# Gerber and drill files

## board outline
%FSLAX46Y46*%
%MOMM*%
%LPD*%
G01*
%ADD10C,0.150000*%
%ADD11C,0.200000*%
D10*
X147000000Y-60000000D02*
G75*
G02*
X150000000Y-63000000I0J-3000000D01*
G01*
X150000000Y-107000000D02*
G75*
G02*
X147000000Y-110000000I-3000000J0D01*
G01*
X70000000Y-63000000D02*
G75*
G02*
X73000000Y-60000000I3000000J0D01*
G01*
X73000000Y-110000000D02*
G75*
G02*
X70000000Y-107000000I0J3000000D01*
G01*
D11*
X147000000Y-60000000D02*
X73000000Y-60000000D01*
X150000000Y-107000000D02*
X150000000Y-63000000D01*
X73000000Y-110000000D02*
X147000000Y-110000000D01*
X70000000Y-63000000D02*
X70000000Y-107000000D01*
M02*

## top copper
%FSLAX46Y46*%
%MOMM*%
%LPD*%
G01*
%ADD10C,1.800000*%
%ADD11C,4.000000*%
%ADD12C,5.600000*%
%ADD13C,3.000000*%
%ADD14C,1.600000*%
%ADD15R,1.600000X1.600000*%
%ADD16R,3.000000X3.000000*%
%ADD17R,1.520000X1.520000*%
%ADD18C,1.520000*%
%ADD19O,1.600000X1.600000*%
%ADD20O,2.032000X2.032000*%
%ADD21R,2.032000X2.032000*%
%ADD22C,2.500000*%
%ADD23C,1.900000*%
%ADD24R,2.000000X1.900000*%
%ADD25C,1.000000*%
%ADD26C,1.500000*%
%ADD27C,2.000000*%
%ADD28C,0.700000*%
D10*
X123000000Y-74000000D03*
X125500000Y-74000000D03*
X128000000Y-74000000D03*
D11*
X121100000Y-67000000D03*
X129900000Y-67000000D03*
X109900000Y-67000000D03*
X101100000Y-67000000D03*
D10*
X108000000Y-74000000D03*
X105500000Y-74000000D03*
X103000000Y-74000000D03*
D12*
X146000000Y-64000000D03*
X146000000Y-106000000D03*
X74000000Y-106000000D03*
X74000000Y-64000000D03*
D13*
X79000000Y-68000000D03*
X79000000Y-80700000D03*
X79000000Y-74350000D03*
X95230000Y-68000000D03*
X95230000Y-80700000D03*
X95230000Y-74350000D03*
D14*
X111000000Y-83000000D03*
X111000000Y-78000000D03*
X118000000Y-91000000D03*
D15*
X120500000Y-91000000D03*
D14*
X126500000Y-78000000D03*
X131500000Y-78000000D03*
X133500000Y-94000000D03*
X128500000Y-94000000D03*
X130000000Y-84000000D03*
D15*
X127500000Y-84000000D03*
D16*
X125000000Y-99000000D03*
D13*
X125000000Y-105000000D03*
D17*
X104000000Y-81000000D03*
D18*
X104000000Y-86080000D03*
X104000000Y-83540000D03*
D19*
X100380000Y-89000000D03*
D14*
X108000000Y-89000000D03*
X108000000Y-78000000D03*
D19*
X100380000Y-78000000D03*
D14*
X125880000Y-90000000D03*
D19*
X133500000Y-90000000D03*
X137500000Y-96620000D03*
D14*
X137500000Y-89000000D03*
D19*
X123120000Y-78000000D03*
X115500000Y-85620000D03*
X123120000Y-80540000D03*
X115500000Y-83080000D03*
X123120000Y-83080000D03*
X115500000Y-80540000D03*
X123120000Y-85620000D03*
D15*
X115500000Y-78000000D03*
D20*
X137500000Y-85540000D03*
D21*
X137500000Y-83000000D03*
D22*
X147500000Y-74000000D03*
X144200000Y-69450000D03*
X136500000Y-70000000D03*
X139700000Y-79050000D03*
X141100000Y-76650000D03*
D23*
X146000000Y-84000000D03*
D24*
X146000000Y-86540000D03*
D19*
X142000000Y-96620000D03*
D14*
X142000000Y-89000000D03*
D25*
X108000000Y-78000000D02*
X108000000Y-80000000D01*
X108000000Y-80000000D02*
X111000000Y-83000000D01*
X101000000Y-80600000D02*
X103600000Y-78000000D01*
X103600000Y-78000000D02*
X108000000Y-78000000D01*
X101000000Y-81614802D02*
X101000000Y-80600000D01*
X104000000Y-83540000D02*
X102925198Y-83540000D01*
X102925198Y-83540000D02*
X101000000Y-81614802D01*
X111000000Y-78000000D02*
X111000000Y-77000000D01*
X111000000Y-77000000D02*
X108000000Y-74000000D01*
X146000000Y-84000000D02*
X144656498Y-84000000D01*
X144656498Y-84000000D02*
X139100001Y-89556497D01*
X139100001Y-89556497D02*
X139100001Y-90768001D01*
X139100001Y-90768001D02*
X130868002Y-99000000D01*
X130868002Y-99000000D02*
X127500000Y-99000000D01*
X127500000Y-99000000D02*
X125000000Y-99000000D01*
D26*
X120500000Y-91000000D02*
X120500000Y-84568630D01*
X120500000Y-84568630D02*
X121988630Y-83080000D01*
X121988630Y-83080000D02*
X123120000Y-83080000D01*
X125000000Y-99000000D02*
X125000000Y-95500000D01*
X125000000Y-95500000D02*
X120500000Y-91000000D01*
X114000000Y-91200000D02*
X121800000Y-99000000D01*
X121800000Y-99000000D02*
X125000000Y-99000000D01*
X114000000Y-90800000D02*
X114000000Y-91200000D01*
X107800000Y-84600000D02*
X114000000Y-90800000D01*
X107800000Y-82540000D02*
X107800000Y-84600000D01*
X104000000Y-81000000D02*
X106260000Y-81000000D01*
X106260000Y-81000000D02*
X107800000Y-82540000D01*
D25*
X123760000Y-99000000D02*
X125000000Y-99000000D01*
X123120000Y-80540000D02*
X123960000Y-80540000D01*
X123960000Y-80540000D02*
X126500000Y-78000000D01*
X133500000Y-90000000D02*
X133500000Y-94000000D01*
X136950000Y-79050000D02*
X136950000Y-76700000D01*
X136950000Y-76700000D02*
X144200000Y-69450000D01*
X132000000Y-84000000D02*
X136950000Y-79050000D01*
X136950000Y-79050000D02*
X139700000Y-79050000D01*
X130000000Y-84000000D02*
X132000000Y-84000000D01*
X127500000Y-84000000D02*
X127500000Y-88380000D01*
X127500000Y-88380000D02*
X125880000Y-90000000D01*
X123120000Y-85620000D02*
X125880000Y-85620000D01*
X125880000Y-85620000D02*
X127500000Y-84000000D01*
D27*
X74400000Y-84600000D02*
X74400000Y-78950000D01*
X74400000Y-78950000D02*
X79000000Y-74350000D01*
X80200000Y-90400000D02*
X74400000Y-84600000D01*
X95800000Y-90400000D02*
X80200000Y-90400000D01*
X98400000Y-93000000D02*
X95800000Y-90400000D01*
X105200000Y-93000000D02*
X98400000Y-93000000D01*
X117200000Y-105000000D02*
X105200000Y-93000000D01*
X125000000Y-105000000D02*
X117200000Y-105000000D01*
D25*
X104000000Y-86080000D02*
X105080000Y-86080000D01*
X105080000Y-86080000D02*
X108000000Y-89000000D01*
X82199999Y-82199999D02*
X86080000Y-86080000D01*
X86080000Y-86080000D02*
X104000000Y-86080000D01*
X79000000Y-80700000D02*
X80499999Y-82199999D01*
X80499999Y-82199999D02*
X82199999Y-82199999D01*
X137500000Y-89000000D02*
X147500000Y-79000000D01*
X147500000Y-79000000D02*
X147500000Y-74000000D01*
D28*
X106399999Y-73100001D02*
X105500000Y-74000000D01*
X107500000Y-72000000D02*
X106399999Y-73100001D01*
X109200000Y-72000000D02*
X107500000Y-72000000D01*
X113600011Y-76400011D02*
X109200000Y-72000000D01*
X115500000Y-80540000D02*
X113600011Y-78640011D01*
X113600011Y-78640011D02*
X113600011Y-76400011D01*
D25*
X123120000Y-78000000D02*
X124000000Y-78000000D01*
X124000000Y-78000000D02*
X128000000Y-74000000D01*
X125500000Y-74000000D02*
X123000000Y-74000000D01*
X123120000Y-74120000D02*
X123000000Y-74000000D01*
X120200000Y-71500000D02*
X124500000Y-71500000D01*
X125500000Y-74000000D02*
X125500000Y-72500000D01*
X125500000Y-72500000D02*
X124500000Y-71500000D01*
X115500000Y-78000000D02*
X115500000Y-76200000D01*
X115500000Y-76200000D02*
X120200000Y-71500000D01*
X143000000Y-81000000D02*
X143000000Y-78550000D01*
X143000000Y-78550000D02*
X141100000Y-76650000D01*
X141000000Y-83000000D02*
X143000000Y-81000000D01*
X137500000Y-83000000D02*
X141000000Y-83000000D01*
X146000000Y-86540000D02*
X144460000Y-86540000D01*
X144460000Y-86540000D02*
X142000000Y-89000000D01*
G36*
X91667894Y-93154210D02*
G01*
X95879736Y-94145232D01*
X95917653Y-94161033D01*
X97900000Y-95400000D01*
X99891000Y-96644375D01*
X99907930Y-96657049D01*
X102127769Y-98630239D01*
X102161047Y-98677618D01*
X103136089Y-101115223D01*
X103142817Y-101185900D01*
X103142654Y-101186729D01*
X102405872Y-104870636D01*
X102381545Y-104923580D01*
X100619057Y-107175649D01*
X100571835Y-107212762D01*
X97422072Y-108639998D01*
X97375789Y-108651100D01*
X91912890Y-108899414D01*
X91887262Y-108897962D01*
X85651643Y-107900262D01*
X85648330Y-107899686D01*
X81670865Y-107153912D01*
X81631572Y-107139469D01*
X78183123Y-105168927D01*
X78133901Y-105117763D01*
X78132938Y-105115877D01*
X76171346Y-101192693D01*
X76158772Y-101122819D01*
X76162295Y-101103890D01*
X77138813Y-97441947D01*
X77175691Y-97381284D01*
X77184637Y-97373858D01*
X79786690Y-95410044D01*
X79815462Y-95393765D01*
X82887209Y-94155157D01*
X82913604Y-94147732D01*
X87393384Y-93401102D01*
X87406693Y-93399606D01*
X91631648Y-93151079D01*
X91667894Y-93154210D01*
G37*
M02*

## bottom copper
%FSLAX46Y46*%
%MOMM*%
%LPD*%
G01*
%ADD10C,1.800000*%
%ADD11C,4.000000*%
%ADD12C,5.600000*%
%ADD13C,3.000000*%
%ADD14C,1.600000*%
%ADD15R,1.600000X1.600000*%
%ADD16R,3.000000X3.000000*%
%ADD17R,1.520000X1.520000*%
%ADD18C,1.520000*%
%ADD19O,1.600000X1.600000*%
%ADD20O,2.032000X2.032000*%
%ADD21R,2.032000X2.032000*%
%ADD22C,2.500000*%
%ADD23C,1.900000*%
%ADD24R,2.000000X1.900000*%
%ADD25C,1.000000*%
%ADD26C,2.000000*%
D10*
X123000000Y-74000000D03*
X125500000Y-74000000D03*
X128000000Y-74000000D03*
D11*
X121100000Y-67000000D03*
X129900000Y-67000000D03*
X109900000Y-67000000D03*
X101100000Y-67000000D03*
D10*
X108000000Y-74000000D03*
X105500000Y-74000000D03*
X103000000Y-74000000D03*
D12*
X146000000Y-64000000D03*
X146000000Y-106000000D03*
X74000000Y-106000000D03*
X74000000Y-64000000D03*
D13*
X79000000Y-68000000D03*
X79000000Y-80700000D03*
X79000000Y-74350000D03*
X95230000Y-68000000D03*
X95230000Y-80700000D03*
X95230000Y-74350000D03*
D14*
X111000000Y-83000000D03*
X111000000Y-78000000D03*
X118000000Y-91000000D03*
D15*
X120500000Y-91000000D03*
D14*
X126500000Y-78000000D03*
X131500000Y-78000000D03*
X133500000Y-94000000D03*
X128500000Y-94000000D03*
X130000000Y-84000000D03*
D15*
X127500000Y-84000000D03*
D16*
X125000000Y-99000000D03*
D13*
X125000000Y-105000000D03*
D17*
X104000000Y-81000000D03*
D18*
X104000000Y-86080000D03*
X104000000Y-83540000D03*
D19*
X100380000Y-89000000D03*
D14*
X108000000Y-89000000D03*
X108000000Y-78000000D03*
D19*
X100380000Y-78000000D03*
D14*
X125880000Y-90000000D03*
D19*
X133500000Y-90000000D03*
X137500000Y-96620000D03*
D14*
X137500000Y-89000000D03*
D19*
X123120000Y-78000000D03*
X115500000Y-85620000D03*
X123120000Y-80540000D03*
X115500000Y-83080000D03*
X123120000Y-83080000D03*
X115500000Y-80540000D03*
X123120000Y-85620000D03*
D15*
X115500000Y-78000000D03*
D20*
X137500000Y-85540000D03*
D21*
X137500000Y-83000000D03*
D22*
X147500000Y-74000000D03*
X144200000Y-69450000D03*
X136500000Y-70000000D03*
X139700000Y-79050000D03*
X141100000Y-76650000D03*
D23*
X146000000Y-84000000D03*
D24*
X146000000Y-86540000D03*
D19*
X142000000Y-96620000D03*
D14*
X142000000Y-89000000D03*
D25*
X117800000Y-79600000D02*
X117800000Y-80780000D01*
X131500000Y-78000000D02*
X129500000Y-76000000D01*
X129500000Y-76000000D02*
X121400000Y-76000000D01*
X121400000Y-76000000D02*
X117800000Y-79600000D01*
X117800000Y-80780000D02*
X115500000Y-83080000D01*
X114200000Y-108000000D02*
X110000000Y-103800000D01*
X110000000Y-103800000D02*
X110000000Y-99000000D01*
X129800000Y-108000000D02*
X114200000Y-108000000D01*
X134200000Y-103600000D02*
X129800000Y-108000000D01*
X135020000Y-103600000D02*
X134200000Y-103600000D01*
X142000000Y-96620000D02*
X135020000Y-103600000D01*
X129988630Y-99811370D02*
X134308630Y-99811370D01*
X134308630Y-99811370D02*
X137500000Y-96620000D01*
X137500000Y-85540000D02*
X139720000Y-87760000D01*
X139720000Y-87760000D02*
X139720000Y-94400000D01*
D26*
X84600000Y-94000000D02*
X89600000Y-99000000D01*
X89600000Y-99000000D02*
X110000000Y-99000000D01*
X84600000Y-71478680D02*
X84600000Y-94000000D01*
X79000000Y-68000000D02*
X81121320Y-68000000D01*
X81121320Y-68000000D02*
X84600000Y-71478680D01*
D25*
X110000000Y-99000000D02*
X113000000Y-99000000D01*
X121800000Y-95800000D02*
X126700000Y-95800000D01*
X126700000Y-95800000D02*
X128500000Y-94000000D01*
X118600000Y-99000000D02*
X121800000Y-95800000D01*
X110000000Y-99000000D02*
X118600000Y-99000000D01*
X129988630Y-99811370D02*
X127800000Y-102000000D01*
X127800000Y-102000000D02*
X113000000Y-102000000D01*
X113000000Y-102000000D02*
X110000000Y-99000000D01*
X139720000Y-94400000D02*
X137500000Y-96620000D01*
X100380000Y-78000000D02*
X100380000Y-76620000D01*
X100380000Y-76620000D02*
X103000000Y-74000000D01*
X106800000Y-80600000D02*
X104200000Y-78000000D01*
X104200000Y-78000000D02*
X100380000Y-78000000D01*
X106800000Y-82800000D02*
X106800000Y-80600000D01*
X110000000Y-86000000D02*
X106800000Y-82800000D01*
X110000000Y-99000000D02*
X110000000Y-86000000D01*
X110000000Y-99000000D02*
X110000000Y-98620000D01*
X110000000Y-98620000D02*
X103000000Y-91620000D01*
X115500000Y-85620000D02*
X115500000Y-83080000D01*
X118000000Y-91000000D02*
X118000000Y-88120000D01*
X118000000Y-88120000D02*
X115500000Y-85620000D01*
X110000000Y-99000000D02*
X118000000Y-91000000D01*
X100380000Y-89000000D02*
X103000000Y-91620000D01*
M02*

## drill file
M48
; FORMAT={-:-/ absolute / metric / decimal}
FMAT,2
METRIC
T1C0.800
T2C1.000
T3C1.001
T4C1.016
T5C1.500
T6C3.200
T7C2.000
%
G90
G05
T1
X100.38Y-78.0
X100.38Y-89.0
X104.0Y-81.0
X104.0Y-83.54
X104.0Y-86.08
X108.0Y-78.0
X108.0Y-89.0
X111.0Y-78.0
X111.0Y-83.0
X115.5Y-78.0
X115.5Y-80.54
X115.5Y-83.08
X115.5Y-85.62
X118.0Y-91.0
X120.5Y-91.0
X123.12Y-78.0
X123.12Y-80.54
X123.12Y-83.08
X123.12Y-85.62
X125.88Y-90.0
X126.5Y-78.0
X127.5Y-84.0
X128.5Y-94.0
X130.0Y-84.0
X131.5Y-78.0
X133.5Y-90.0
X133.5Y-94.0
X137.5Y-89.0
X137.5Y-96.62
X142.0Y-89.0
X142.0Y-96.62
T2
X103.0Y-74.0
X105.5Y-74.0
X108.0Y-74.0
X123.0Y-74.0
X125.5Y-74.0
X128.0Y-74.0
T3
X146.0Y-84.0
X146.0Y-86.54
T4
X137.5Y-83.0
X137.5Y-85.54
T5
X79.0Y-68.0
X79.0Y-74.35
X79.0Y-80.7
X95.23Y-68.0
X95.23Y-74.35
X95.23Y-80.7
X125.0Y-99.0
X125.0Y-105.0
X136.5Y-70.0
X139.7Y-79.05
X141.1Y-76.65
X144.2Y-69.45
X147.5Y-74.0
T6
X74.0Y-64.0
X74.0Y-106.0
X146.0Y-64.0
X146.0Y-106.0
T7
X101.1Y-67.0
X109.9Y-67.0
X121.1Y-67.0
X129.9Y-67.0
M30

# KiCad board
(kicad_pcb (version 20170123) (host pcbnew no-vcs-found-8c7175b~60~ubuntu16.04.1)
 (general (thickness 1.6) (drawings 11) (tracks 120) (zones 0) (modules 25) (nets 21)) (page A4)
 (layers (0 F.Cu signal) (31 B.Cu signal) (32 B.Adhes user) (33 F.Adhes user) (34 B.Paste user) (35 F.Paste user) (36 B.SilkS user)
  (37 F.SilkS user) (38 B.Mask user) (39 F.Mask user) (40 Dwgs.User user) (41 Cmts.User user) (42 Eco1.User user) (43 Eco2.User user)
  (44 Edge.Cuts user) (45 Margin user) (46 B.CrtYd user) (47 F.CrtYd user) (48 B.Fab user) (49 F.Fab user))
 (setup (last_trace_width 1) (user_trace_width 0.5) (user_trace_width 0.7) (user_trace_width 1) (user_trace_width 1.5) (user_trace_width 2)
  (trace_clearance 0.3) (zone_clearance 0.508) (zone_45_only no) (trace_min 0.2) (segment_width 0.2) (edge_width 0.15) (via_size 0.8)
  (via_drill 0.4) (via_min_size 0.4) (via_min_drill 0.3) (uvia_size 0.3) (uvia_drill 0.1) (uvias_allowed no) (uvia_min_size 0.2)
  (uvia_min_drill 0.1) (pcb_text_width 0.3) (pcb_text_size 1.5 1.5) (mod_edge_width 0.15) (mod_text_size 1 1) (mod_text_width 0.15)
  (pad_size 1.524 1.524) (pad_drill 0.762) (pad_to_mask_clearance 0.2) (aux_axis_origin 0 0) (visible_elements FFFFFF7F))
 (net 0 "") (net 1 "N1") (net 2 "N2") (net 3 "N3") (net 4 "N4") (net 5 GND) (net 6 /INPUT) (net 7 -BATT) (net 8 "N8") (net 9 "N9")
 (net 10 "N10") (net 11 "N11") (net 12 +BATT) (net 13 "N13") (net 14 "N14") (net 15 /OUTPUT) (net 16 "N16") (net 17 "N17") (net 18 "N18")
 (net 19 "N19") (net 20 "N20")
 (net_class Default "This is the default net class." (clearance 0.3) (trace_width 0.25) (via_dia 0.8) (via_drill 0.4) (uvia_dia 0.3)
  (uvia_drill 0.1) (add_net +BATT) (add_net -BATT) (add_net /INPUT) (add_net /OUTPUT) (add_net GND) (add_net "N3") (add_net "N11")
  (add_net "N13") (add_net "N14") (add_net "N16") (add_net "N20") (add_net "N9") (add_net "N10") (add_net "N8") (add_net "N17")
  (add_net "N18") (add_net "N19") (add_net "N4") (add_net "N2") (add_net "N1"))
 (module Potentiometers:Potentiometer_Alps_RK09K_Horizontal (layer F.Cu) (at 128 74 90)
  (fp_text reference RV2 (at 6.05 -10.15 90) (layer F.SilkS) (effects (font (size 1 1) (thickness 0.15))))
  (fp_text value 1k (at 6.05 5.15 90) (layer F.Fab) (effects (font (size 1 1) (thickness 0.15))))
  (pad 3 thru_hole circle (at 0 -5 90) (size 1.8 1.8) (drill 1) (layers *.Cu *.Mask) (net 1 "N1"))
  (pad 2 thru_hole circle (at 0 -2.5 90) (size 1.8 1.8) (drill 1) (layers *.Cu *.Mask) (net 1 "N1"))
  (pad 1 thru_hole circle (at 0 0 90) (size 1.8 1.8) (drill 1) (layers *.Cu *.Mask) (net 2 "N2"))
  (pad 0 np_thru_hole circle (at 7 -6.9 90) (size 4 4) (drill 2) (layers *.Cu *.Mask))
  (pad 0 np_thru_hole circle (at 7 1.9 90) (size 4 4) (drill 2) (layers *.Cu *.Mask)))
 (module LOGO (layer F.Cu) (at 89.9 101.4)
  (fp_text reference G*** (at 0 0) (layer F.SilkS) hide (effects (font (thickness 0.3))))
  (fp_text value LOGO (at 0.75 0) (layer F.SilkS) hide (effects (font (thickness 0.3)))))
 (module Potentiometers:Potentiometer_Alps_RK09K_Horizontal (layer F.Cu) (at 108 74 90)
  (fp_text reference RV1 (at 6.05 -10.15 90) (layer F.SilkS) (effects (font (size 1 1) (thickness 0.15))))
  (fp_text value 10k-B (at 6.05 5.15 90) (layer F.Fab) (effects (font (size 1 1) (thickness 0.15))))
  (pad 0 np_thru_hole circle (at 7 1.9 90) (size 4 4) (drill 2) (layers *.Cu *.Mask))
  (pad 0 np_thru_hole circle (at 7 -6.9 90) (size 4 4) (drill 2) (layers *.Cu *.Mask))
  (pad 1 thru_hole circle (at 0 0 90) (size 1.8 1.8) (drill 1) (layers *.Cu *.Mask) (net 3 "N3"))
  (pad 2 thru_hole circle (at 0 -2.5 90) (size 1.8 1.8) (drill 1) (layers *.Cu *.Mask) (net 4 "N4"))
  (pad 3 thru_hole circle (at 0 -5 90) (size 1.8 1.8) (drill 1) (layers *.Cu *.Mask) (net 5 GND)))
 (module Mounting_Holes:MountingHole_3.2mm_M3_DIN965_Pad (layer F.Cu) (at 146 64)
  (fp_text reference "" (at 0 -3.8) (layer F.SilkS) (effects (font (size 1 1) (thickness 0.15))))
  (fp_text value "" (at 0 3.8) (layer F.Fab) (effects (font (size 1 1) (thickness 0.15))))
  (pad 1 thru_hole circle (at 0 0) (size 5.6 5.6) (drill 3.2) (layers *.Cu *.Mask)))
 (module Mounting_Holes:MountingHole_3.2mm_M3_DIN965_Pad (layer F.Cu) (at 146 106)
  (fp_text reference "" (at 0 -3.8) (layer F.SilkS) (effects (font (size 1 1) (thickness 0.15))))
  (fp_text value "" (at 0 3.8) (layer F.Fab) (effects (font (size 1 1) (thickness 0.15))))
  (pad 1 thru_hole circle (at 0 0) (size 5.6 5.6) (drill 3.2) (layers *.Cu *.Mask)))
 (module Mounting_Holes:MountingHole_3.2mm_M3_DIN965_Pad (layer F.Cu) (at 74 106)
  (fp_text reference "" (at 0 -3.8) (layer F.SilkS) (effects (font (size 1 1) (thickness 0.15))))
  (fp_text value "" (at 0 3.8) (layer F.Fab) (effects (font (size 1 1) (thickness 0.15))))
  (pad 1 thru_hole circle (at 0 0) (size 5.6 5.6) (drill 3.2) (layers *.Cu *.Mask)))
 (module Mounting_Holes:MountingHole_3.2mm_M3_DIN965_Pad (layer F.Cu) (at 74 64)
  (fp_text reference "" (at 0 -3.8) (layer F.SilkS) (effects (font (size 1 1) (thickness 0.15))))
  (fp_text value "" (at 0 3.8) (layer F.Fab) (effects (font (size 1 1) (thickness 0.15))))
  (pad 1 thru_hole circle (at 0 0) (size 5.6 5.6) (drill 3.2) (layers *.Cu *.Mask)))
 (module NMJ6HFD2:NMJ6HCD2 (layer F.Cu) (at 79 68)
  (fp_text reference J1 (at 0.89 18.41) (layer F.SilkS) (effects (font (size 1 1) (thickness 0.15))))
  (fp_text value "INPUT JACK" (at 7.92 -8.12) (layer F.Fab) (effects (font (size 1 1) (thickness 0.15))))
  (pad 3 thru_hole circle (at 0 0) (size 3 3) (drill 1.5) (layers *.Cu *.Mask) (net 5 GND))
  (pad 1 thru_hole circle (at 0 12.7) (size 3 3) (drill 1.5) (layers *.Cu *.Mask) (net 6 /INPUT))
  (pad 2 thru_hole circle (at 0 6.35) (size 3 3) (drill 1.5) (layers *.Cu *.Mask) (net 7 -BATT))
  (pad 6 thru_hole circle (at 16.23 0) (size 3 3) (drill 1.5) (layers *.Cu *.Mask) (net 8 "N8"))
  (pad 4 thru_hole circle (at 16.23 12.7) (size 3 3) (drill 1.5) (layers *.Cu *.Mask) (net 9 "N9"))
  (pad 5 thru_hole circle (at 16.23 6.35) (size 3 3) (drill 1.5) (layers *.Cu *.Mask) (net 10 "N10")))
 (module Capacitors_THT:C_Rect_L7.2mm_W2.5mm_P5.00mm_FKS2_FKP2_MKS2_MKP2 (layer F.Cu) (at 111 78 270)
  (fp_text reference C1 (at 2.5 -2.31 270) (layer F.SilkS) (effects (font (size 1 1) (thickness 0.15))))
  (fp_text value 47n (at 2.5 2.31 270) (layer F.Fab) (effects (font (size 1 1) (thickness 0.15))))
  (pad 2 thru_hole circle (at 5 0 270) (size 1.6 1.6) (drill 0.8) (layers *.Cu *.Mask) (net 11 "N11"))
  (pad 1 thru_hole circle (at 0 0 270) (size 1.6 1.6) (drill 0.8) (layers *.Cu *.Mask) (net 3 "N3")))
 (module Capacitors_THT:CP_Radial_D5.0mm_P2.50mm (layer F.Cu) (at 120.5 91 180)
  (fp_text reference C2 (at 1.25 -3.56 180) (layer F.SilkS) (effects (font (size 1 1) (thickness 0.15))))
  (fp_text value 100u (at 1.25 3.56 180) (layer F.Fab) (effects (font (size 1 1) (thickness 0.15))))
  (pad 2 thru_hole circle (at 2.5 0 180) (size 1.6 1.6) (drill 0.8) (layers *.Cu *.Mask) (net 5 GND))
  (pad 1 thru_hole rect (at 0 0 180) (size 1.6 1.6) (drill 0.8) (layers *.Cu *.Mask) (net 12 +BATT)))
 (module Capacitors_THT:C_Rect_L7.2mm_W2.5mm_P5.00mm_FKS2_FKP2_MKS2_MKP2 (layer F.Cu) (at 131.5 78 180)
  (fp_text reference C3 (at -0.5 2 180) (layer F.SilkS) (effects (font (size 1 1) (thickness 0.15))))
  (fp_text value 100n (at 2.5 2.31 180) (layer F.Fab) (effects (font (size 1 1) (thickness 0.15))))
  (pad 2 thru_hole circle (at 5 0 180) (size 1.6 1.6) (drill 0.8) (layers *.Cu *.Mask) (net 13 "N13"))
  (pad 1 thru_hole circle (at 0 0 180) (size 1.6 1.6) (drill 0.8) (layers *.Cu *.Mask) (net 5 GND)))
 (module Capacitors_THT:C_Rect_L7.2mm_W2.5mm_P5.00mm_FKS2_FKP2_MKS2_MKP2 (layer F.Cu) (at 133.5 94 180)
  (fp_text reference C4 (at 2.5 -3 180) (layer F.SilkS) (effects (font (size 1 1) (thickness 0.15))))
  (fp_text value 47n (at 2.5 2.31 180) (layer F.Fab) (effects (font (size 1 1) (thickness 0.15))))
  (pad 1 thru_hole circle (at 0 0 180) (size 1.6 1.6) (drill 0.8) (layers *.Cu *.Mask) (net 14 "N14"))
  (pad 2 thru_hole circle (at 5 0 180) (size 1.6 1.6) (drill 0.8) (layers *.Cu *.Mask) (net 5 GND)))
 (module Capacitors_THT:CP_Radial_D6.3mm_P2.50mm (layer F.Cu) (at 127.5 84)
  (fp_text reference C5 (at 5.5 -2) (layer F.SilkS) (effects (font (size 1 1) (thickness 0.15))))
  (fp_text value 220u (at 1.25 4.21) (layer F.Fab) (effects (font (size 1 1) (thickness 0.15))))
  (pad 2 thru_hole circle (at 2.5 0) (size 1.6 1.6) (drill 0.8) (layers *.Cu *.Mask) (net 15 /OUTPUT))
  (pad 1 thru_hole rect (at 0 0) (size 1.6 1.6) (drill 0.8) (layers *.Cu *.Mask) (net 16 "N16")))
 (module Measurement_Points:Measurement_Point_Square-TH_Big (layer F.Cu) (at 125 99)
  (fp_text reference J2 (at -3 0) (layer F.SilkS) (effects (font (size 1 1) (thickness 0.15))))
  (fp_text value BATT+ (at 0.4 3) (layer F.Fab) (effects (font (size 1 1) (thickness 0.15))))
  (pad 1 thru_hole rect (at 0 0) (size 3 3) (drill 1.5) (layers *.Cu *.Mask) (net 12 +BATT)))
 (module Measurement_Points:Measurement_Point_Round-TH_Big (layer F.Cu) (at 125 105)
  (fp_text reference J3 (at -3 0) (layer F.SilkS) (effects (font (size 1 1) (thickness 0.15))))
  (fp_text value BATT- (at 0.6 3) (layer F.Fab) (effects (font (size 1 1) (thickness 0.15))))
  (pad 1 thru_hole circle (at 0 0) (size 3 3) (drill 1.5) (layers *.Cu *.Mask) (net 7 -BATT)))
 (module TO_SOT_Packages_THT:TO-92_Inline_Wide (layer F.Cu) (at 104 81 270)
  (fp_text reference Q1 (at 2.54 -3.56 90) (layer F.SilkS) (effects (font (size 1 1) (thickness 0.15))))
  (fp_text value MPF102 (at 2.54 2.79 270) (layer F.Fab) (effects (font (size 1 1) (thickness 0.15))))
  (pad 1 thru_hole rect (at 0 0) (size 1.52 1.52) (drill 0.8) (layers *.Cu *.Mask) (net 12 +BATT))
  (pad 3 thru_hole circle (at 5.08 0) (size 1.52 1.52) (drill 0.8) (layers *.Cu *.Mask) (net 6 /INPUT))
  (pad 2 thru_hole circle (at 2.54 0) (size 1.52 1.52) (drill 0.8) (layers *.Cu *.Mask) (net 11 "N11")))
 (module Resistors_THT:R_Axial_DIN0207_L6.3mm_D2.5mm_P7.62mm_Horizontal (layer F.Cu) (at 108 89 180)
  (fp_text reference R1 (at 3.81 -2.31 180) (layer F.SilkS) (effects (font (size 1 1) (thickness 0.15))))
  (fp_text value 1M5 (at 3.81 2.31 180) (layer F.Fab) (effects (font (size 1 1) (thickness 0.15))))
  (pad 2 thru_hole oval (at 7.62 0 180) (size 1.6 1.6) (drill 0.8) (layers *.Cu *.Mask) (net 5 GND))
  (pad 1 thru_hole circle (at 0 0 180) (size 1.6 1.6) (drill 0.8) (layers *.Cu *.Mask) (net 6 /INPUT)))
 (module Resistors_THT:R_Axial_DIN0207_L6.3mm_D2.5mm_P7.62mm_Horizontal (layer F.Cu) (at 108 78 180)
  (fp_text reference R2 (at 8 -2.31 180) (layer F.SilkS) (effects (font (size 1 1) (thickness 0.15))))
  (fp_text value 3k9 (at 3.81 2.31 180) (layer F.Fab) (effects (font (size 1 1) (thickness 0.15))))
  (pad 1 thru_hole circle (at 0 0 180) (size 1.6 1.6) (drill 0.8) (layers *.Cu *.Mask) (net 11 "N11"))
  (pad 2 thru_hole oval (at 7.62 0 180) (size 1.6 1.6) (drill 0.8) (layers *.Cu *.Mask) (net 5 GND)))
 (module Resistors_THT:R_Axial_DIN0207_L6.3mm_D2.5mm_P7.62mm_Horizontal (layer F.Cu) (at 125.88 90)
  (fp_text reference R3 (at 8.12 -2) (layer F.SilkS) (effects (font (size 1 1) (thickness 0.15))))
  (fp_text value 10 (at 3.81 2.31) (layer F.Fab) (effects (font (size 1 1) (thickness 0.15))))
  (pad 1 thru_hole circle (at 0 0) (size 1.6 1.6) (drill 0.8) (layers *.Cu *.Mask) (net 16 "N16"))
  (pad 2 thru_hole oval (at 7.62 0) (size 1.6 1.6) (drill 0.8) (layers *.Cu *.Mask) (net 14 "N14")))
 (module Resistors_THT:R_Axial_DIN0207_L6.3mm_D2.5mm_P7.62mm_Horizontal (layer F.Cu) (at 137.5 89 270)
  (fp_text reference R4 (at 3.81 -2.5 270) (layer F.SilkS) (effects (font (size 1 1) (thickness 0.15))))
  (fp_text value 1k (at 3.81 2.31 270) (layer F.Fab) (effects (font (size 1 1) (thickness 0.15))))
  (pad 2 thru_hole oval (at 7.62 0 270) (size 1.6 1.6) (drill 0.8) (layers *.Cu *.Mask) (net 5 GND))
  (pad 1 thru_hole circle (at 0 0 270) (size 1.6 1.6) (drill 0.8) (layers *.Cu *.Mask) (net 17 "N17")))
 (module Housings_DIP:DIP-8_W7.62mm (layer F.Cu) (at 115.5 78)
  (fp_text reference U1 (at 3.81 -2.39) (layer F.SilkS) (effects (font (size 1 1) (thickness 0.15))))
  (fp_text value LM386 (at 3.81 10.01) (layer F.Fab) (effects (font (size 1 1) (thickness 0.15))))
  (pad 8 thru_hole oval (at 7.62 0) (size 1.6 1.6) (drill 0.8) (layers *.Cu *.Mask) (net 2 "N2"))
  (pad 4 thru_hole oval (at 0 7.62) (size 1.6 1.6) (drill 0.8) (layers *.Cu *.Mask) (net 5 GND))
  (pad 7 thru_hole oval (at 7.62 2.54) (size 1.6 1.6) (drill 0.8) (layers *.Cu *.Mask) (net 13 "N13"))
  (pad 3 thru_hole oval (at 0 5.08) (size 1.6 1.6) (drill 0.8) (layers *.Cu *.Mask) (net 5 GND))
  (pad 6 thru_hole oval (at 7.62 5.08) (size 1.6 1.6) (drill 0.8) (layers *.Cu *.Mask) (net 12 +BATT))
  (pad 2 thru_hole oval (at 0 2.54) (size 1.6 1.6) (drill 0.8) (layers *.Cu *.Mask) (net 4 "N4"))
  (pad 5 thru_hole oval (at 7.62 7.62) (size 1.6 1.6) (drill 0.8) (layers *.Cu *.Mask) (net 16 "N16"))
  (pad 1 thru_hole rect (at 0 0) (size 1.6 1.6) (drill 0.8) (layers *.Cu *.Mask) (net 1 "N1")))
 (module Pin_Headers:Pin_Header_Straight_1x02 (layer F.Cu) (at 137.5 83)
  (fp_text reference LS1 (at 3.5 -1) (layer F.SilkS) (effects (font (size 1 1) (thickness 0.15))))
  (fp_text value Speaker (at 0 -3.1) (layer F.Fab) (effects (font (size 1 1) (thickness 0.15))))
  (pad 2 thru_hole oval (at 0 2.54) (size 2.032 2.032) (drill 1.016) (layers *.Cu *.Mask) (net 5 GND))
  (pad 1 thru_hole rect (at 0 0) (size 2.032 2.032) (drill 1.016) (layers *.Cu *.Mask) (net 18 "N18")))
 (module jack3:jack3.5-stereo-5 (layer F.Cu) (at 147.5 74 270)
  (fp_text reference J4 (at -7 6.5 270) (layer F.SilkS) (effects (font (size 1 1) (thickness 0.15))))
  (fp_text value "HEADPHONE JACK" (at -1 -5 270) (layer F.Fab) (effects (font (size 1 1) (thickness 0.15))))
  (pad 3 thru_hole circle (at 0 0 270) (size 2.5 2.5) (drill 1.5) (layers *.Cu *.Mask) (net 17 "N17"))
  (pad 1 thru_hole circle (at -4.55 3.3 270) (size 2.5 2.5) (drill 1.5) (layers *.Cu *.Mask) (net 15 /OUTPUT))
  (pad 5 thru_hole circle (at -4 11 270) (size 2.5 2.5) (drill 1.5) (layers *.Cu *.Mask) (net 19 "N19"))
  (pad 2 thru_hole circle (at 5.05 7.8 270) (size 2.5 2.5) (drill 1.5) (layers *.Cu *.Mask) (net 15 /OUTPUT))
  (pad 4 thru_hole circle (at 2.65 6.4 270) (size 2.5 2.5) (drill 1.5) (layers *.Cu *.Mask) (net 18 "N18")))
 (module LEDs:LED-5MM (layer F.Cu) (at 146 86.54 90)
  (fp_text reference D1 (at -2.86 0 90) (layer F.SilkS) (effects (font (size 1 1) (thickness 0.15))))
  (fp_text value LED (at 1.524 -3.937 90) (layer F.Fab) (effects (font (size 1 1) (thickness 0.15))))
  (pad 2 thru_hole circle (at 2.54 0 90) (size 1.9 1.9) (drill 1.00076) (layers *.Cu *.Mask) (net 12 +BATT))
  (pad 1 thru_hole rect (at 0 0 180) (size 2 1.9) (drill 1.00076) (layers *.Cu *.Mask) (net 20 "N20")))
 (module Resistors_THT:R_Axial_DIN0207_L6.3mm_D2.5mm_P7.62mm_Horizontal (layer F.Cu) (at 142 89 270)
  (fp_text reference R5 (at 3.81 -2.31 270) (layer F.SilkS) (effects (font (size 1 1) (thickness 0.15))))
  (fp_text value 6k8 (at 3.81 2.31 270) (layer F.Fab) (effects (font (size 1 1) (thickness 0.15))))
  (pad 2 thru_hole oval (at 7.62 0 270) (size 1.6 1.6) (drill 0.8) (layers *.Cu *.Mask) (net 5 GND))
  (pad 1 thru_hole circle (at 0 0 270) (size 1.6 1.6) (drill 0.8) (layers *.Cu *.Mask) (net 20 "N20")))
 (gr_arc (start 147 63) (end 150 63) (angle -90) (layer Edge.Cuts) (width 0.15))
 (gr_arc (start 147 107) (end 147 110) (angle -90) (layer Edge.Cuts) (width 0.15))
 (gr_arc (start 73 63) (end 73 60) (angle -90) (layer Edge.Cuts) (width 0.15))
 (gr_arc (start 73 107) (end 70 107) (angle -90) (layer Edge.Cuts) (width 0.15))
 (gr_line (start 147 60) (end 73 60) (layer Edge.Cuts) (width 0.2))
 (gr_line (start 150 107) (end 150 63) (layer Edge.Cuts) (width 0.2))
 (gr_line (start 73 110) (end 147 110) (layer Edge.Cuts) (width 0.2))
 (gr_line (start 70 63) (end 70 107) (layer Edge.Cuts) (width 0.2))
 (segment (start 108 78) (end 108 80) (width 1) (layer F.Cu) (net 11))
 (segment (start 108 80) (end 111 83) (width 1) (layer F.Cu) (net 11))
 (segment (start 101 80.6) (end 103.6 78) (width 1) (layer F.Cu) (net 11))
 (segment (start 103.6 78) (end 108 78) (width 1) (layer F.Cu) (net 11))
 (segment (start 101 81.614802) (end 101 80.6) (width 1) (layer F.Cu) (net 11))
 (segment (start 104 83.54) (end 102.925198 83.54) (width 1) (layer F.Cu) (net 11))
 (segment (start 102.925198 83.54) (end 101 81.614802) (width 1) (layer F.Cu) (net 11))
 (segment (start 111 78) (end 111 77) (width 1) (layer F.Cu) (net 3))
 (segment (start 111 77) (end 108 74) (width 1) (layer F.Cu) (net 3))
 (segment (start 117.8 79.6) (end 117.8 80.78) (width 1) (layer B.Cu) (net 5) (status 1000000))
 (segment (start 131.5 78) (end 129.5 76) (width 1) (layer B.Cu) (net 5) (status 1000000))
 (segment (start 129.5 76) (end 121.4 76) (width 1) (layer B.Cu) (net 5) (status 1000000))
 (segment (start 121.4 76) (end 117.8 79.6) (width 1) (layer B.Cu) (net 5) (status 1000000))
 (segment (start 117.8 80.78) (end 115.5 83.08) (width 1) (layer B.Cu) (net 5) (status 1000000))
 (segment (start 114.2 108) (end 110 103.8) (width 1) (layer B.Cu) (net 5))
 (segment (start 110 103.8) (end 110 99) (width 1) (layer B.Cu) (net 5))
 (segment (start 129.8 108) (end 114.2 108) (width 1) (layer B.Cu) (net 5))
 (segment (start 134.2 103.6) (end 129.8 108) (width 1) (layer B.Cu) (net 5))
 (segment (start 135.02 103.6) (end 134.2 103.6) (width 1) (layer B.Cu) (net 5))
 (segment (start 142 96.62) (end 135.02 103.6) (width 1) (layer B.Cu) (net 5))
 (segment (start 129.98863 99.81137) (end 134.30863 99.81137) (width 1) (layer B.Cu) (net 5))
 (segment (start 134.30863 99.81137) (end 137.5 96.62) (width 1) (layer B.Cu) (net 5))
 (segment (start 137.5 85.54) (end 139.72 87.76) (width 1) (layer B.Cu) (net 5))
 (segment (start 139.72 87.76) (end 139.72 94.4) (width 1) (layer B.Cu) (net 5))
 (segment (start 84.6 94) (end 89.6 99) (width 2) (layer B.Cu) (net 5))
 (segment (start 89.6 99) (end 110 99) (width 2) (layer B.Cu) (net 5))
 (segment (start 84.6 71.47868) (end 84.6 94) (width 2) (layer B.Cu) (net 5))
 (segment (start 79 68) (end 81.12132 68) (width 2) (layer B.Cu) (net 5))
 (segment (start 81.12132 68) (end 84.6 71.47868) (width 2) (layer B.Cu) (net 5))
 (segment (start 110 99) (end 113 99) (width 1) (layer B.Cu) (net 5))
 (segment (start 121.8 95.8) (end 126.7 95.8) (width 1) (layer B.Cu) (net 5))
 (segment (start 126.7 95.8) (end 128.5 94) (width 1) (layer B.Cu) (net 5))
 (segment (start 118.6 99) (end 121.8 95.8) (width 1) (layer B.Cu) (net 5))
 (segment (start 110 99) (end 118.6 99) (width 1) (layer B.Cu) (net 5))
 (segment (start 129.98863 99.81137) (end 127.8 102) (width 1) (layer B.Cu) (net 5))
 (segment (start 127.8 102) (end 113 102) (width 1) (layer B.Cu) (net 5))
 (segment (start 113 102) (end 110 99) (width 1) (layer B.Cu) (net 5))
 (segment (start 139.72 94.4) (end 137.5 96.62) (width 1) (layer B.Cu) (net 5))
 (segment (start 100.38 78) (end 100.38 76.62) (width 1) (layer B.Cu) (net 5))
 (segment (start 100.38 76.62) (end 103 74) (width 1) (layer B.Cu) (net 5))
 (segment (start 106.8 80.6) (end 104.2 78) (width 1) (layer B.Cu) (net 5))
 (segment (start 104.2 78) (end 100.38 78) (width 1) (layer B.Cu) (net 5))
 (segment (start 106.8 82.8) (end 106.8 80.6) (width 1) (layer B.Cu) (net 5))
 (segment (start 110 86) (end 106.8 82.8) (width 1) (layer B.Cu) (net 5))
 (segment (start 110 99) (end 110 86) (width 1) (layer B.Cu) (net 5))
 (segment (start 110 99) (end 110 98.62) (width 1) (layer B.Cu) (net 5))
 (segment (start 110 98.62) (end 103 91.62) (width 1) (layer B.Cu) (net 5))
 (segment (start 115.5 85.62) (end 115.5 83.08) (width 1) (layer B.Cu) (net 5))
 (segment (start 118 91) (end 118 88.12) (width 1) (layer B.Cu) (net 5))
 (segment (start 118 88.12) (end 115.5 85.62) (width 1) (layer B.Cu) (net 5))
 (segment (start 110 99) (end 118 91) (width 1) (layer B.Cu) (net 5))
 (segment (start 100.38 89) (end 103 91.62) (width 1) (layer B.Cu) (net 5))
 (segment (start 146 84) (end 144.656498 84) (width 1) (layer F.Cu) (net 12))
 (segment (start 144.656498 84) (end 139.100001 89.556497) (width 1) (layer F.Cu) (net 12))
 (segment (start 139.100001 89.556497) (end 139.100001 90.768001) (width 1) (layer F.Cu) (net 12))
 (segment (start 139.100001 90.768001) (end 130.868002 99) (width 1) (layer F.Cu) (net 12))
 (segment (start 130.868002 99) (end 127.5 99) (width 1) (layer F.Cu) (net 12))
 (segment (start 127.5 99) (end 125 99) (width 1) (layer F.Cu) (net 12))
 (segment (start 120.5 91) (end 120.5 84.56863) (width 1.5) (layer F.Cu) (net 12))
 (segment (start 120.5 84.56863) (end 121.98863 83.08) (width 1.5) (layer F.Cu) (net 12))
 (segment (start 121.98863 83.08) (end 123.12 83.08) (width 1.5) (layer F.Cu) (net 12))
 (segment (start 125 99) (end 125 95.5) (width 1.5) (layer F.Cu) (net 12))
 (segment (start 125 95.5) (end 120.5 91) (width 1.5) (layer F.Cu) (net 12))
 (segment (start 114 91.2) (end 121.8 99) (width 1.5) (layer F.Cu) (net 12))
 (segment (start 121.8 99) (end 125 99) (width 1.5) (layer F.Cu) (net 12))
 (segment (start 114 90.8) (end 114 91.2) (width 1.5) (layer F.Cu) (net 12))
 (segment (start 107.8 84.6) (end 114 90.8) (width 1.5) (layer F.Cu) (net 12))
 (segment (start 107.8 82.54) (end 107.8 84.6) (width 1.5) (layer F.Cu) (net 12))
 (segment (start 104 81) (end 106.26 81) (width 1.5) (layer F.Cu) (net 12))
 (segment (start 106.26 81) (end 107.8 82.54) (width 1.5) (layer F.Cu) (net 12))
 (segment (start 123.76 99) (end 125 99) (width 1) (layer F.Cu) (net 12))
 (segment (start 123.12 80.54) (end 123.96 80.54) (width 1) (layer F.Cu) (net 13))
 (segment (start 123.96 80.54) (end 126.5 78) (width 1) (layer F.Cu) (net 13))
 (segment (start 133.5 90) (end 133.5 94) (width 1) (layer F.Cu) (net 14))
 (segment (start 136.95 79.05) (end 136.95 76.7) (width 1) (layer F.Cu) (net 15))
 (segment (start 136.95 76.7) (end 144.2 69.45) (width 1) (layer F.Cu) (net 15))
 (segment (start 132 84) (end 136.95 79.05) (width 1) (layer F.Cu) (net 15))
 (segment (start 136.95 79.05) (end 139.7 79.05) (width 1) (layer F.Cu) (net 15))
 (segment (start 130 84) (end 132 84) (width 1) (layer F.Cu) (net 15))
 (segment (start 127.5 84) (end 127.5 88.38) (width 1) (layer F.Cu) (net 16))
 (segment (start 127.5 88.38) (end 125.88 90) (width 1) (layer F.Cu) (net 16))
 (segment (start 123.12 85.62) (end 125.88 85.62) (width 1) (layer F.Cu) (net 16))
 (segment (start 125.88 85.62) (end 127.5 84) (width 1) (layer F.Cu) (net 16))
 (segment (start 74.4 84.6) (end 74.4 78.95) (width 2) (layer F.Cu) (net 7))
 (segment (start 74.4 78.95) (end 79 74.35) (width 2) (layer F.Cu) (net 7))
 (segment (start 80.2 90.4) (end 74.4 84.6) (width 2) (layer F.Cu) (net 7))
 (segment (start 95.8 90.4) (end 80.2 90.4) (width 2) (layer F.Cu) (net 7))
 (segment (start 98.4 93) (end 95.8 90.4) (width 2) (layer F.Cu) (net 7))
 (segment (start 105.2 93) (end 98.4 93) (width 2) (layer F.Cu) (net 7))
 (segment (start 117.2 105) (end 105.2 93) (width 2) (layer F.Cu) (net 7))
 (segment (start 125 105) (end 117.2 105) (width 2) (layer F.Cu) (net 7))
 (segment (start 104 86.08) (end 105.08 86.08) (width 1) (layer F.Cu) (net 6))
 (segment (start 105.08 86.08) (end 108 89) (width 1) (layer F.Cu) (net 6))
 (segment (start 82.199999 82.199999) (end 86.08 86.08) (width 1) (layer F.Cu) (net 6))
 (segment (start 86.08 86.08) (end 104 86.08) (width 1) (layer F.Cu) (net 6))
 (segment (start 79 80.7) (end 80.499999 82.199999) (width 1) (layer F.Cu) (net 6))
 (segment (start 80.499999 82.199999) (end 82.199999 82.199999) (width 1) (layer F.Cu) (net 6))
 (segment (start 137.5 89) (end 147.5 79) (width 1) (layer F.Cu) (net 17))
 (segment (start 147.5 79) (end 147.5 74) (width 1) (layer F.Cu) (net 17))
 (segment (start 106.399999 73.100001) (end 105.5 74) (width 0.7) (layer F.Cu) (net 4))
 (segment (start 107.5 72) (end 106.399999 73.100001) (width 0.7) (layer F.Cu) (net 4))
 (segment (start 109.2 72) (end 107.5 72) (width 0.7) (layer F.Cu) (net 4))
 (segment (start 113.600011 76.400011) (end 109.2 72) (width 0.7) (layer F.Cu) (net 4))
 (segment (start 115.5 80.54) (end 113.600011 78.640011) (width 0.7) (layer F.Cu) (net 4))
 (segment (start 113.600011 78.640011) (end 113.600011 76.400011) (width 0.7) (layer F.Cu) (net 4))
 (segment (start 123.12 78) (end 124 78) (width 1) (layer F.Cu) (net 2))
 (segment (start 124 78) (end 128 74) (width 1) (layer F.Cu) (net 2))
 (segment (start 125.5 74) (end 123 74) (width 1) (layer F.Cu) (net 1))
 (segment (start 123.12 74.12) (end 123 74) (width 1) (layer F.Cu) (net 1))
 (segment (start 120.2 71.5) (end 124.5 71.5) (width 1) (layer F.Cu) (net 1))
 (segment (start 125.5 74) (end 125.5 72.5) (width 1) (layer F.Cu) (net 1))
 (segment (start 125.5 72.5) (end 124.5 71.5) (width 1) (layer F.Cu) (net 1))
 (segment (start 115.5 78) (end 115.5 76.2) (width 1) (layer F.Cu) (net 1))
 (segment (start 115.5 76.2) (end 120.2 71.5) (width 1) (layer F.Cu) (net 1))
 (segment (start 143 81) (end 143 78.55) (width 1) (layer F.Cu) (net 18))
 (segment (start 143 78.55) (end 141.1 76.65) (width 1) (layer F.Cu) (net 18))
 (segment (start 141 83) (end 143 81) (width 1) (layer F.Cu) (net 18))
 (segment (start 137.5 83) (end 141 83) (width 1) (layer F.Cu) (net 18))
 (segment (start 146 86.54) (end 144.46 86.54) (width 1) (layer F.Cu) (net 20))
 (segment (start 144.46 86.54) (end 142 89) (width 1) (layer F.Cu) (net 20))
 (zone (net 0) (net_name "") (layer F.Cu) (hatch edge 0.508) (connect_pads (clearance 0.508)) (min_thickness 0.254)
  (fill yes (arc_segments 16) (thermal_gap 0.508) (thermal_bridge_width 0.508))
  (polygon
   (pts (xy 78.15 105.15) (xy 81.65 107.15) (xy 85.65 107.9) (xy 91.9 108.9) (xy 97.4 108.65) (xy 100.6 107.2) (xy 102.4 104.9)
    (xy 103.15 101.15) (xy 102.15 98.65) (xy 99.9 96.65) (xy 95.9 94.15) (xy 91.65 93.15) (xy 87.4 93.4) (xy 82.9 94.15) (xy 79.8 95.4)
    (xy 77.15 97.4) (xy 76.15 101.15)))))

